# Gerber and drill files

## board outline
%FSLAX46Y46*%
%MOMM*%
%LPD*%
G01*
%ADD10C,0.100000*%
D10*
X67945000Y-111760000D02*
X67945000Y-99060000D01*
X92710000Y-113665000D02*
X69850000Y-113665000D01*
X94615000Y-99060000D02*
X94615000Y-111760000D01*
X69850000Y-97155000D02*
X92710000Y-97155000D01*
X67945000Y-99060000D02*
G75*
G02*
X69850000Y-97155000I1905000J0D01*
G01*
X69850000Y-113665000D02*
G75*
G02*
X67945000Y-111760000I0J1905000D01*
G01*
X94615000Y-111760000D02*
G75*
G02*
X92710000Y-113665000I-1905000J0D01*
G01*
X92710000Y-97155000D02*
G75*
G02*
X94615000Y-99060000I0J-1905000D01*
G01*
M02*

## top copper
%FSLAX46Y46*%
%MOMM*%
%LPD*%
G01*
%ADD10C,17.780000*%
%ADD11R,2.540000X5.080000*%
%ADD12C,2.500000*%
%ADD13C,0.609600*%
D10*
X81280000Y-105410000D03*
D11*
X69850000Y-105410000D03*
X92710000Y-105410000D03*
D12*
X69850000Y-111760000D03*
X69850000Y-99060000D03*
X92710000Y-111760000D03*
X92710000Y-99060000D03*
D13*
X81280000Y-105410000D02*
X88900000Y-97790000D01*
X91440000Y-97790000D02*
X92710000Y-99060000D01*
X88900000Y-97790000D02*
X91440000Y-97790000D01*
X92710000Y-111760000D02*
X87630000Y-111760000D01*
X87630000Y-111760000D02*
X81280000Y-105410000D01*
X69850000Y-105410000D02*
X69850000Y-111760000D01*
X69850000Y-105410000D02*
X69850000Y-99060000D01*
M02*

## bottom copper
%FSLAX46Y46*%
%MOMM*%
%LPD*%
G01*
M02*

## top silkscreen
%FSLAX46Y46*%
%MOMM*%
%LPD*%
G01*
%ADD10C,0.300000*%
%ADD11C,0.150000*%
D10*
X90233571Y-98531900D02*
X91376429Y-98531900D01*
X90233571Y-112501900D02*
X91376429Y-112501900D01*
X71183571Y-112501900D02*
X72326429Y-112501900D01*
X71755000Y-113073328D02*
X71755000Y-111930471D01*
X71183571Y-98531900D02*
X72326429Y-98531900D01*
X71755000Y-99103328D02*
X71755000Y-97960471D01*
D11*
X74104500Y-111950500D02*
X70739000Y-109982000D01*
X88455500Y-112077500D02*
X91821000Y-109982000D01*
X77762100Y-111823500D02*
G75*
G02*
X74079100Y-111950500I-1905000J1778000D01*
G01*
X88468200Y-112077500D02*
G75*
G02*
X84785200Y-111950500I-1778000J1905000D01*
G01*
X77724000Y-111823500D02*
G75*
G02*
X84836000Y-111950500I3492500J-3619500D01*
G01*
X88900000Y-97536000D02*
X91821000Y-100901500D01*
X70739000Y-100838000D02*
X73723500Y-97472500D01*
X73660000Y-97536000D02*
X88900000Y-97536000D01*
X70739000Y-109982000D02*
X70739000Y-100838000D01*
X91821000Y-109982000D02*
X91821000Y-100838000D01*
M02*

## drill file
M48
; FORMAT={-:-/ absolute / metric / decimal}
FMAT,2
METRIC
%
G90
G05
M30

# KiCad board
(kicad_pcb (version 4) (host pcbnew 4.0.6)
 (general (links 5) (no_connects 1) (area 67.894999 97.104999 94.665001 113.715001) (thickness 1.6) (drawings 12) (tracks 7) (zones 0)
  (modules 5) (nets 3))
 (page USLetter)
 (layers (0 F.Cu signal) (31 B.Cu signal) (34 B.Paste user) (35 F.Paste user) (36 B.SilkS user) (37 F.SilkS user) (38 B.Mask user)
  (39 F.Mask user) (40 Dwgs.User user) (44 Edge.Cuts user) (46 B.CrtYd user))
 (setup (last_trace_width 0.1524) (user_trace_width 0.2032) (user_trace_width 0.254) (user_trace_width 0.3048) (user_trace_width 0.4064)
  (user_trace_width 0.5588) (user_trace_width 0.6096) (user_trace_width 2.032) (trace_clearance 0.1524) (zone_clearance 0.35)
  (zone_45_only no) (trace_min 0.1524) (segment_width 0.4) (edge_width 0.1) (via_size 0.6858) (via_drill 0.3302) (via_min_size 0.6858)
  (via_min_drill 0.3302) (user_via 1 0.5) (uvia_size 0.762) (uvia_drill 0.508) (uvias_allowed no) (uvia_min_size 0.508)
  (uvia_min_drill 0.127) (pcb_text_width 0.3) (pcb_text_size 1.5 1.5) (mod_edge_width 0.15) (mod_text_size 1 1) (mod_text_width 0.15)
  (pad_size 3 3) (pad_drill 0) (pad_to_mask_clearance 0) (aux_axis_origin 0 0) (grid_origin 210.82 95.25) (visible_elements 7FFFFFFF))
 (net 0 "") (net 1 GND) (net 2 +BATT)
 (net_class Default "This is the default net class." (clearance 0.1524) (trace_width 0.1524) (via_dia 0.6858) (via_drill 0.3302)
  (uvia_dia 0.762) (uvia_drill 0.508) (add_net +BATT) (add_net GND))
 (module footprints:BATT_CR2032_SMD (layer F.Cu) (at 81.28 105.41)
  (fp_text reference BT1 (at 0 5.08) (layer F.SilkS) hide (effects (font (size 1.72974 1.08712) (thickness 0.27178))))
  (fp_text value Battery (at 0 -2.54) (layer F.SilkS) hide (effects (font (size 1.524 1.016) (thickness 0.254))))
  (fp_line (start -7.1755 6.5405) (end -10.541 4.572) (layer F.SilkS) (width 0.15))
  (fp_line (start 7.1755 6.6675) (end 10.541 4.572) (layer F.SilkS) (width 0.15))
  (fp_arc (start -5.4229 4.6355) (end -3.5179 6.4135) (angle 90) (layer F.SilkS) (width 0.15))
  (fp_arc (start 5.4102 4.7625) (end 7.1882 6.6675) (angle 90) (layer F.SilkS) (width 0.15))
  (fp_arc (start -0.0635 10.033) (end -3.556 6.4135) (angle 90) (layer F.SilkS) (width 0.15))
  (fp_line (start 7.62 -7.874) (end 10.541 -4.5085) (layer F.SilkS) (width 0.15))
  (fp_line (start -10.541 -4.572) (end -7.5565 -7.9375) (layer F.SilkS) (width 0.15))
  (fp_line (start -7.62 -7.874) (end 7.62 -7.874) (layer F.SilkS) (width 0.15))
  (fp_line (start -10.541 4.572) (end -10.541 -4.572) (layer F.SilkS) (width 0.15))
  (fp_line (start 10.541 4.572) (end 10.541 -4.572) (layer F.SilkS) (width 0.15))
  (pad 2 smd circle (at 0 0) (size 17.78 17.78) (layers F.Cu F.Paste F.Mask) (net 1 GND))
  (pad 1 smd rect (at -11.43 0) (size 2.54 5.08) (layers F.Cu F.Paste F.Mask) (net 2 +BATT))
  (pad 1 smd rect (at 11.43 0) (size 2.54 5.08) (layers F.Cu F.Paste F.Mask) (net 2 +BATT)))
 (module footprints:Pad (layer F.Cu) (at 69.85 111.76)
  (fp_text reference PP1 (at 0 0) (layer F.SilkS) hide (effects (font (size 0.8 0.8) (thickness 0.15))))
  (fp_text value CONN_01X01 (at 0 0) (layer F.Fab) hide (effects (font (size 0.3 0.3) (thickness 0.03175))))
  (pad 1 smd circle (at 0 0) (size 2.5 2.5) (layers F.Cu F.Paste F.Mask) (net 2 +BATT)))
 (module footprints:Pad (layer F.Cu) (at 69.85 99.06)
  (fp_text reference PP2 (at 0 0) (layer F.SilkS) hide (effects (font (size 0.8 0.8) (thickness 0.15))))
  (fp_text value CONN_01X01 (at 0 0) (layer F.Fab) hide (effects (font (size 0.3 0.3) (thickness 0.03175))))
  (pad 1 smd circle (at 0 0) (size 2.5 2.5) (layers F.Cu F.Paste F.Mask) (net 2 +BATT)))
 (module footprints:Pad (layer F.Cu) (at 92.71 111.76)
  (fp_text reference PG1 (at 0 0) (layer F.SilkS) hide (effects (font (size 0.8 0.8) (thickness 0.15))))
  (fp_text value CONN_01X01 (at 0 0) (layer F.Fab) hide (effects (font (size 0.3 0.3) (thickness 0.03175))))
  (pad 1 smd circle (at 0 0) (size 2.5 2.5) (layers F.Cu F.Paste F.Mask) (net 1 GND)))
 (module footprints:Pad (layer F.Cu) (at 92.71 99.06)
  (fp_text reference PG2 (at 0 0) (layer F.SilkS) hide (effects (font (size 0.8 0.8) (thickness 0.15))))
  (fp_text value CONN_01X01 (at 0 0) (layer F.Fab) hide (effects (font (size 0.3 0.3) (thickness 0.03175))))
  (pad 1 smd circle (at 0 0) (size 2.5 2.5) (layers F.Cu F.Paste F.Mask) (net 1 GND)))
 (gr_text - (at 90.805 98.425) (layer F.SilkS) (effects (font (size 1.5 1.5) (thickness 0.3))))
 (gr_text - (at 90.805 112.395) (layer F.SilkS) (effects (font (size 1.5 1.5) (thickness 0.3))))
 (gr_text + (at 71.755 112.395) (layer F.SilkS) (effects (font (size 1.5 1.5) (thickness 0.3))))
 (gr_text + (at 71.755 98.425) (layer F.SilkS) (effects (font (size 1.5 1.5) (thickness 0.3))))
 (gr_line (start 67.945 111.76) (end 67.945 99.06) (angle 90) (layer Edge.Cuts) (width 0.1))
 (gr_line (start 92.71 113.665) (end 69.85 113.665) (angle 90) (layer Edge.Cuts) (width 0.1))
 (gr_line (start 94.615 99.06) (end 94.615 111.76) (angle 90) (layer Edge.Cuts) (width 0.1))
 (gr_line (start 69.85 97.155) (end 92.71 97.155) (angle 90) (layer Edge.Cuts) (width 0.1))
 (gr_arc (start 69.85 99.06) (end 67.945 99.06) (angle 90) (layer Edge.Cuts) (width 0.1))
 (gr_arc (start 69.85 111.76) (end 69.85 113.665) (angle 90) (layer Edge.Cuts) (width 0.1))
 (gr_arc (start 92.71 111.76) (end 94.615 111.76) (angle 90) (layer Edge.Cuts) (width 0.1))
 (gr_arc (start 92.71 99.06) (end 92.71 97.155) (angle 90) (layer Edge.Cuts) (width 0.1))
 (segment (start 81.28 105.41) (end 88.9 97.79) (width 0.6096) (layer F.Cu) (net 1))
 (segment (start 91.44 97.79) (end 92.71 99.06) (width 0.6096) (layer F.Cu) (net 1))
 (segment (start 88.9 97.79) (end 91.44 97.79) (width 0.6096) (layer F.Cu) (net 1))
 (segment (start 92.71 111.76) (end 87.63 111.76) (width 0.6096) (layer F.Cu) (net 1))
 (segment (start 87.63 111.76) (end 81.28 105.41) (width 0.6096) (layer F.Cu) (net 1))
 (segment (start 69.85 105.41) (end 69.85 111.76) (width 0.6096) (layer F.Cu) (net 2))
 (segment (start 69.85 105.41) (end 69.85 99.06) (width 0.6096) (layer F.Cu) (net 2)))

